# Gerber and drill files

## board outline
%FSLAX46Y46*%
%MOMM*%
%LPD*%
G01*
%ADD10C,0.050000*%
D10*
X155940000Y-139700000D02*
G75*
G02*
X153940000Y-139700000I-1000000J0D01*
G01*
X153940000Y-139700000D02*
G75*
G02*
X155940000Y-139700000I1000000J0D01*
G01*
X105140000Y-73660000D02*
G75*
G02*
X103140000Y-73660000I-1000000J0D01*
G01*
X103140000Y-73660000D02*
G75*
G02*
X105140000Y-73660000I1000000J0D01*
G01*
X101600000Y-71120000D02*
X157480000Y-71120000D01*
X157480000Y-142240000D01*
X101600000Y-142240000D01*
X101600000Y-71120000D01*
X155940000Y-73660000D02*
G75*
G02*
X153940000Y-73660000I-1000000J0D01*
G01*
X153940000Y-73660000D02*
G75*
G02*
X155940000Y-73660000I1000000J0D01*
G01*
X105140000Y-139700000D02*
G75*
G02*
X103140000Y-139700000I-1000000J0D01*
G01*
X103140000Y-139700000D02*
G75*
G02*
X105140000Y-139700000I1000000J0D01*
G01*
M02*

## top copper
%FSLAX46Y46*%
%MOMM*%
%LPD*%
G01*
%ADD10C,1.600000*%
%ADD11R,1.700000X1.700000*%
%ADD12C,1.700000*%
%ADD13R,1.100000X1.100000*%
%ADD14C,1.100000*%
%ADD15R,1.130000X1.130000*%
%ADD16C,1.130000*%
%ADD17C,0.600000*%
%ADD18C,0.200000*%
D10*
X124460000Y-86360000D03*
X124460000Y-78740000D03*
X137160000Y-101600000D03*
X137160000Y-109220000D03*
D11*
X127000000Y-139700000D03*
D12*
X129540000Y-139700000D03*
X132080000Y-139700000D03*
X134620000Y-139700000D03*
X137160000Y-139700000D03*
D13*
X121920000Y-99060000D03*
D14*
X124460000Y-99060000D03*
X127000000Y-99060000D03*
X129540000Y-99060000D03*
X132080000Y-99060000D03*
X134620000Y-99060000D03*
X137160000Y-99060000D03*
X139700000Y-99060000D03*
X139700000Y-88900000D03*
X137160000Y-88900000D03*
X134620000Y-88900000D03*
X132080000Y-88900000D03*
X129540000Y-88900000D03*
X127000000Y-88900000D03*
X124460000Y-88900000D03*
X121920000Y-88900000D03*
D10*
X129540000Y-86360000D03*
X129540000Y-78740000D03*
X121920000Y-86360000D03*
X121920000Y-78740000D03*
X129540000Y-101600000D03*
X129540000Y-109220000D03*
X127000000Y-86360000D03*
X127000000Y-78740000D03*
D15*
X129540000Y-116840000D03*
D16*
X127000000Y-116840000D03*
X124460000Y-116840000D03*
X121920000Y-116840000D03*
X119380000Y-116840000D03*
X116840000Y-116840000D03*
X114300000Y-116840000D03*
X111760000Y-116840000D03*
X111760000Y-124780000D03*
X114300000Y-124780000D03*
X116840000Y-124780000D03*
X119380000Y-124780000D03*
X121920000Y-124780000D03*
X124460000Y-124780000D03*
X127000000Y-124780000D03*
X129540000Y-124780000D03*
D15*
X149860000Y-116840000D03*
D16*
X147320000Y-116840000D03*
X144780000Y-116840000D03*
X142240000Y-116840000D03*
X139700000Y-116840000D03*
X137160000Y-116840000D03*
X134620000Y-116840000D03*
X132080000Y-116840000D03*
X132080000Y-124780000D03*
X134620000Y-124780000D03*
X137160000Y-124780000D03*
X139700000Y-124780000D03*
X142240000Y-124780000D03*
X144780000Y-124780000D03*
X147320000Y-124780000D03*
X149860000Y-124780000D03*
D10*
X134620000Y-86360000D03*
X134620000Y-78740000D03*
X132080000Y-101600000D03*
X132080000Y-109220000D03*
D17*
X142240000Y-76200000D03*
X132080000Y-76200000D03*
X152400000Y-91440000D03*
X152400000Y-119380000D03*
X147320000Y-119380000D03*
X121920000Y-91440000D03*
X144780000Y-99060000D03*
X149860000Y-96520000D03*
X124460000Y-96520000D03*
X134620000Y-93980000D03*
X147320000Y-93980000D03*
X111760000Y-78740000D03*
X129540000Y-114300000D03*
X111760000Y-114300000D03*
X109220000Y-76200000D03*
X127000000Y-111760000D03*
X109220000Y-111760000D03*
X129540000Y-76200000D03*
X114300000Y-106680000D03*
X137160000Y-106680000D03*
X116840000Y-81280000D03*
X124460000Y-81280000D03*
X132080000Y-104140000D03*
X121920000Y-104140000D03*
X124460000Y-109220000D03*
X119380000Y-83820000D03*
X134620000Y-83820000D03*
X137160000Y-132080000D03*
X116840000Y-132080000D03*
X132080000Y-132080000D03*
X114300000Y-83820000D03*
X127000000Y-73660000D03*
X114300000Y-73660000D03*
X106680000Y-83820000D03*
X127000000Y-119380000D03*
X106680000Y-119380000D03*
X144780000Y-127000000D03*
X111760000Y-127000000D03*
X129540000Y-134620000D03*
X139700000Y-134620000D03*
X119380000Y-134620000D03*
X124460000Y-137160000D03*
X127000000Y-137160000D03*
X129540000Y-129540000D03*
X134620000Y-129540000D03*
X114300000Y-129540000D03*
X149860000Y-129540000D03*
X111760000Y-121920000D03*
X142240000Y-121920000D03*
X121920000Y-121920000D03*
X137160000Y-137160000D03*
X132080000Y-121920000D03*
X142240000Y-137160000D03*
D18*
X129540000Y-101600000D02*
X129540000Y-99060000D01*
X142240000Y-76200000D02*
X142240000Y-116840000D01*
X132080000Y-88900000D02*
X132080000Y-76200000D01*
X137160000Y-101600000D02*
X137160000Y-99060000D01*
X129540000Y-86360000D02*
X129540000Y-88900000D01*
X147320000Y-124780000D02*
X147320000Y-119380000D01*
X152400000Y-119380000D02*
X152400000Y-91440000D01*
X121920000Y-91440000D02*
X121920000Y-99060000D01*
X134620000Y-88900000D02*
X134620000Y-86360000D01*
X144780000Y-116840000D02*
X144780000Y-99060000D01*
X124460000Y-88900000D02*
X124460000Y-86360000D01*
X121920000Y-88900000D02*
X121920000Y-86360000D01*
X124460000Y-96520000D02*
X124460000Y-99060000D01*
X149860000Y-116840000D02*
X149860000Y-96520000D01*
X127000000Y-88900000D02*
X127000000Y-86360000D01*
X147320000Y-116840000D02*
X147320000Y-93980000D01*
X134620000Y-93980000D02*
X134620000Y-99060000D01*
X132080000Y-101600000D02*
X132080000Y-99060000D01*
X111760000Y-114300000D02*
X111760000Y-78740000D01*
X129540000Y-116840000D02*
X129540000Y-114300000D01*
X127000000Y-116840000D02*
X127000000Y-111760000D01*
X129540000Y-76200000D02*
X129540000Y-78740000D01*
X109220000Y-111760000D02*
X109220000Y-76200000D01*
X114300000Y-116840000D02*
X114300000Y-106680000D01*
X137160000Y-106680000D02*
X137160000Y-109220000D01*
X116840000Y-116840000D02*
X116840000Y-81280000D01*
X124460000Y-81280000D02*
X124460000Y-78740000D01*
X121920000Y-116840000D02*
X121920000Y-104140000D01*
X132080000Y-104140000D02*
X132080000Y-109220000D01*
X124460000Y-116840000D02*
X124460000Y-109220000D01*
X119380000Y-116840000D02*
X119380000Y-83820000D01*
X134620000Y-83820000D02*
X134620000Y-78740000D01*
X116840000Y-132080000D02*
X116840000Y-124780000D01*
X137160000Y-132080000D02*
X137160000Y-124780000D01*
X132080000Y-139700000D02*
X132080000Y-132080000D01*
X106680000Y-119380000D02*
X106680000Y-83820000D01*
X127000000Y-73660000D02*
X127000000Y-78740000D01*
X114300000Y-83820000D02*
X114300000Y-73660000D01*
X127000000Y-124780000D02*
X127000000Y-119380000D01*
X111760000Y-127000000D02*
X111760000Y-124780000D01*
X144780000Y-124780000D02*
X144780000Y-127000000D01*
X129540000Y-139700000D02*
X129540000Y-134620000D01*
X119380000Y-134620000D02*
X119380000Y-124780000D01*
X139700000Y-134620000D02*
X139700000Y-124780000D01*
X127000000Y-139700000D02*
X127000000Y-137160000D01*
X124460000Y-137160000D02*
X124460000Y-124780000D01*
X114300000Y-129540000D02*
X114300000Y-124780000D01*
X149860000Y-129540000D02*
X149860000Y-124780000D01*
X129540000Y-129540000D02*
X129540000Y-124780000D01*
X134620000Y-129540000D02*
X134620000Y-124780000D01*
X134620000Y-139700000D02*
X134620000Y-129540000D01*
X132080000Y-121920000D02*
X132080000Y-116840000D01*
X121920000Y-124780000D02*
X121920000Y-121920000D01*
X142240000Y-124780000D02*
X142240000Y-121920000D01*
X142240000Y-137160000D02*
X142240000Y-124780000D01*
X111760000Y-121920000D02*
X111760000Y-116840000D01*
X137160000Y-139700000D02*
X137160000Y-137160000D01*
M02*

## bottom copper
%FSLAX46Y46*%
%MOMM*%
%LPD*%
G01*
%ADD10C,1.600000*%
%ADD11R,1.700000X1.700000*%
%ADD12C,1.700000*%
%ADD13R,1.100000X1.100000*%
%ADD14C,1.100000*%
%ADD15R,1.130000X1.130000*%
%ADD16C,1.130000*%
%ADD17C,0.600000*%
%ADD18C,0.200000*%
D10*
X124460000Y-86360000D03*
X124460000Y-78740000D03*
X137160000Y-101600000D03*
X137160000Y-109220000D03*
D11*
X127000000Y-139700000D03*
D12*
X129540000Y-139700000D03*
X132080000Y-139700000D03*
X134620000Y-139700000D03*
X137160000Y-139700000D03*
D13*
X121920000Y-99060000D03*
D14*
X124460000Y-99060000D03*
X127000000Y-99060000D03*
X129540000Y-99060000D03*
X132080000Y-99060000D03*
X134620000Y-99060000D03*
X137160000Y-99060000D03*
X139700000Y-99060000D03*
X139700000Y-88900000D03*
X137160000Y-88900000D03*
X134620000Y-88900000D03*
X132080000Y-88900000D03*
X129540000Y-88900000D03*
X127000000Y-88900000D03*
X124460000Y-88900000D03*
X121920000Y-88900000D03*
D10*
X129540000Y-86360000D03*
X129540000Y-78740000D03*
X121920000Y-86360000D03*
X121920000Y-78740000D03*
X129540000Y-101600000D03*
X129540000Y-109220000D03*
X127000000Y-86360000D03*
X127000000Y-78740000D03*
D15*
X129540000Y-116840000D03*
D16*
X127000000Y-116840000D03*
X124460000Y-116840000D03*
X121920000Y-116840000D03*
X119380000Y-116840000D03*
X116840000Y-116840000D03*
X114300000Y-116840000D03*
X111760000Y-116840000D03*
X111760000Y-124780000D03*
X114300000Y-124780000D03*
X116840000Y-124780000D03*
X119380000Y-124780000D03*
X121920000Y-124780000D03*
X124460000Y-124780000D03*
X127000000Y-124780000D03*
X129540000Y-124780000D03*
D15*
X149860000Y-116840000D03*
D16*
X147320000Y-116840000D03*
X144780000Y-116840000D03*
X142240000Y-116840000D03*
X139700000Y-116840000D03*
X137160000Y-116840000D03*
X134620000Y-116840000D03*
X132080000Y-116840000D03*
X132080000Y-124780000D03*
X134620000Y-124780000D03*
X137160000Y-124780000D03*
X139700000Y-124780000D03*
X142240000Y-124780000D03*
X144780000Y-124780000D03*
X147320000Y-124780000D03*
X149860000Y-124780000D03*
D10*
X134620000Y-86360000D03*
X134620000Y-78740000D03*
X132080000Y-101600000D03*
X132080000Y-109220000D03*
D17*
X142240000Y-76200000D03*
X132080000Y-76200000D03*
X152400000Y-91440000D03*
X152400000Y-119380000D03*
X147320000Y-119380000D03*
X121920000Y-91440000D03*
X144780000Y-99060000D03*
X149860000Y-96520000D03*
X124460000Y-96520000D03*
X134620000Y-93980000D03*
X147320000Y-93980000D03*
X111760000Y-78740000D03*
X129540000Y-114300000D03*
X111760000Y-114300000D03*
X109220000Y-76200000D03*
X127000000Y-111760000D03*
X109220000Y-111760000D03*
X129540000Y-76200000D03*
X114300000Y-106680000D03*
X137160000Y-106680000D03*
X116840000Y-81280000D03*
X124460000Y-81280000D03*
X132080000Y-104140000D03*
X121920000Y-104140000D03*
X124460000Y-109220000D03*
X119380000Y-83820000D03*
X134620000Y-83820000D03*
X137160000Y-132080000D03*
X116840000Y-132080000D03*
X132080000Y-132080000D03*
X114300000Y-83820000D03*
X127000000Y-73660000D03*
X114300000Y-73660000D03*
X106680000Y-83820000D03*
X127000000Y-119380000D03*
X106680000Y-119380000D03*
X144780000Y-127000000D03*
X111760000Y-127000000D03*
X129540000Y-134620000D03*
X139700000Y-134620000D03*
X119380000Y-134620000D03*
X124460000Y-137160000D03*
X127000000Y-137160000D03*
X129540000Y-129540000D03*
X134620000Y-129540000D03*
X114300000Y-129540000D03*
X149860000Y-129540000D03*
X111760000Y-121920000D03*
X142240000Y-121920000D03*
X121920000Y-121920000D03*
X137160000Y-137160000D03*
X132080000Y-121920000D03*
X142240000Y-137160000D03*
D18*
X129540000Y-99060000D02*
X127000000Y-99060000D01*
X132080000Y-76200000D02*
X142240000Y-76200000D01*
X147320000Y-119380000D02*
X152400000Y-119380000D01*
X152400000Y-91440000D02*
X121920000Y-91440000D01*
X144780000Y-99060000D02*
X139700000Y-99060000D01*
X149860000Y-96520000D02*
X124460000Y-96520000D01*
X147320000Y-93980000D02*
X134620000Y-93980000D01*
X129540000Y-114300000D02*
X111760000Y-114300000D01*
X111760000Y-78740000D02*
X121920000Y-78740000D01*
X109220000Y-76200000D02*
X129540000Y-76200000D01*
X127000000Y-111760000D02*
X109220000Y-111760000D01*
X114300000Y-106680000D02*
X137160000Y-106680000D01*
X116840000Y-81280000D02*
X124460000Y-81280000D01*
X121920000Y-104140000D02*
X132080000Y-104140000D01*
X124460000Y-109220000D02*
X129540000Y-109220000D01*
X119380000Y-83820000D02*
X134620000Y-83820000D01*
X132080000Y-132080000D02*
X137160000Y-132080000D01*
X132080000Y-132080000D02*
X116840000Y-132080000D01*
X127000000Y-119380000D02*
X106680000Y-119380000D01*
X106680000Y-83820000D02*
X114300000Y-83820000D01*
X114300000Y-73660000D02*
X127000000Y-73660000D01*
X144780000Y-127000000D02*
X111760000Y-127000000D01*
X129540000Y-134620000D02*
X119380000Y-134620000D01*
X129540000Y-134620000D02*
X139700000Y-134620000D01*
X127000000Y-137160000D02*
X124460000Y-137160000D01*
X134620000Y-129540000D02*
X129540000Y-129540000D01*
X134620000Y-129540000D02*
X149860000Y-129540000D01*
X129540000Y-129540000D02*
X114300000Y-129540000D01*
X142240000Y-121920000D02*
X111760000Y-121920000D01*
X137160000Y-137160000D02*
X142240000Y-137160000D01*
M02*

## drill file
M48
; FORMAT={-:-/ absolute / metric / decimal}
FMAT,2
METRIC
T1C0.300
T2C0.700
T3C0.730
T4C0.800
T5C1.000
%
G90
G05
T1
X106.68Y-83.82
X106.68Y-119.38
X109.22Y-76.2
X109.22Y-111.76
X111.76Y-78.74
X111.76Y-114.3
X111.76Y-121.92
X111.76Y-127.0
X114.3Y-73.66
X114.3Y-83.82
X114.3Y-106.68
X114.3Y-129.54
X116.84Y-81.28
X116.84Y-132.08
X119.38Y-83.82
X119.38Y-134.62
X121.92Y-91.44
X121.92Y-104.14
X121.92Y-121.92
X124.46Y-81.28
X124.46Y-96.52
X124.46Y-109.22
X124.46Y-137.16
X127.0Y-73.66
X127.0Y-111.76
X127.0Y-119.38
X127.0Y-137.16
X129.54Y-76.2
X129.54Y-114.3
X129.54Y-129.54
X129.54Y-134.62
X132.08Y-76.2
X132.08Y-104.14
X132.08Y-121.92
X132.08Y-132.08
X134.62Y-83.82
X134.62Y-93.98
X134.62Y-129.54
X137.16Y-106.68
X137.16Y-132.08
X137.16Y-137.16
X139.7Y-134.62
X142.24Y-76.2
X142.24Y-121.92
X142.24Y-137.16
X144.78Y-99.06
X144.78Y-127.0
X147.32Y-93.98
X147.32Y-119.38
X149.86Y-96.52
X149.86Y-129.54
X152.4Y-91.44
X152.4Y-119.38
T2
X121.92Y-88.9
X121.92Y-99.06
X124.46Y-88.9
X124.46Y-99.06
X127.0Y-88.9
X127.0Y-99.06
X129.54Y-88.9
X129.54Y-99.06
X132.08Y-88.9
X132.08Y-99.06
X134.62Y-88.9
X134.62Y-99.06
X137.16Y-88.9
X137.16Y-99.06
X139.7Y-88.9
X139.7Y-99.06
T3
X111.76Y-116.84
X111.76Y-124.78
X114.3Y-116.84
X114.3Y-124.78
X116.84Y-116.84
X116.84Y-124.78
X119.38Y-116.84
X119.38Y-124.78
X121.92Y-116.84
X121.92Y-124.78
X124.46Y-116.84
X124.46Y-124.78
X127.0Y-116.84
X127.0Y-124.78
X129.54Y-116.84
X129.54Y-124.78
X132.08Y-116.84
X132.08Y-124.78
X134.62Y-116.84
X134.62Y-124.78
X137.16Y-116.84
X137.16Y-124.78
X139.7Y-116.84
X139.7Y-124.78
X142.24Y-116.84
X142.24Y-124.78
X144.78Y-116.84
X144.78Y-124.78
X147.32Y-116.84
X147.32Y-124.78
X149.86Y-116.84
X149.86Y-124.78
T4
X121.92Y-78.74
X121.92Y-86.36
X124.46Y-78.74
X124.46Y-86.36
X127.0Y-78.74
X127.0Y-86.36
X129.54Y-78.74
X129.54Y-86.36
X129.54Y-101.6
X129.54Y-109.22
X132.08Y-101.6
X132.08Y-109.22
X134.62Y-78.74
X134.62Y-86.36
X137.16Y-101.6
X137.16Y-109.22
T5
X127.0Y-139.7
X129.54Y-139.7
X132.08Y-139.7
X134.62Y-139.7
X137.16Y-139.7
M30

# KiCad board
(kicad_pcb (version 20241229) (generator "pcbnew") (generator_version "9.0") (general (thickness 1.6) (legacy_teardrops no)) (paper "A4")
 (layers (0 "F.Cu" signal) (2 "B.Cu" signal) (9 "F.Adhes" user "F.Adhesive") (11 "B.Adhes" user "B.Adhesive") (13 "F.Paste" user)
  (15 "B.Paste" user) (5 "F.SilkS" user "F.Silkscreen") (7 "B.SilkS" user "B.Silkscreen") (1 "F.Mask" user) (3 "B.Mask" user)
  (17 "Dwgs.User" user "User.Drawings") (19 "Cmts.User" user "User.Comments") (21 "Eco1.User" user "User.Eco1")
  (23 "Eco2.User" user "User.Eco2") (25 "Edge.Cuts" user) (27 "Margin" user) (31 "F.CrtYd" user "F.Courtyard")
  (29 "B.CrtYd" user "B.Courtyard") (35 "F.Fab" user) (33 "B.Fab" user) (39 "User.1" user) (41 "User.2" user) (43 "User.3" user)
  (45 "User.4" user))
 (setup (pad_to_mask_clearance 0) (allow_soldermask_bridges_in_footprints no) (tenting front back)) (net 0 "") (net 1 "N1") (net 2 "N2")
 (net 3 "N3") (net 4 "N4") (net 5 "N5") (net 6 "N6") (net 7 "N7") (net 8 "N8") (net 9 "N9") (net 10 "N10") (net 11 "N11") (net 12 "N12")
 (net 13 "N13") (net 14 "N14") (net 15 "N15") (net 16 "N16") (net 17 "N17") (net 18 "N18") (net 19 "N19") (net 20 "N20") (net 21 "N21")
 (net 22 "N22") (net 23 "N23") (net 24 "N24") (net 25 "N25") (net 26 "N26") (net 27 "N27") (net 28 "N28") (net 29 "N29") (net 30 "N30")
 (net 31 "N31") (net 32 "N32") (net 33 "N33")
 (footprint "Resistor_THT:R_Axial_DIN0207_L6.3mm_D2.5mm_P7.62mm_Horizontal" (layer "F.Cu") (at 124.46 86.36 90)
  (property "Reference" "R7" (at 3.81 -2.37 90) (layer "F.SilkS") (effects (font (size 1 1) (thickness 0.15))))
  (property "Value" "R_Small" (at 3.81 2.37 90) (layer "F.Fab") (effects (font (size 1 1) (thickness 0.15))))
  (pad "1" thru_hole circle (at 0 0 90) (size 1.6 1.6) (drill 0.8) (layers "*.Cu" "*.Mask") (remove_unused_layers no) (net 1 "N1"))
  (pad "2" thru_hole circle (at 7.62 0 90) (size 1.6 1.6) (drill 0.8) (layers "*.Cu" "*.Mask") (remove_unused_layers no) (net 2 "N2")))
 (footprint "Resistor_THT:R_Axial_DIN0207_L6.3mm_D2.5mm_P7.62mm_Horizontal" (layer "F.Cu") (at 137.16 101.6 -90)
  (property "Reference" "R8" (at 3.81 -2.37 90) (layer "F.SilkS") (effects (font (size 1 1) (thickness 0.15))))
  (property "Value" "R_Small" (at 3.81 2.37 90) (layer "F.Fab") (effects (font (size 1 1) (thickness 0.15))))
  (pad "1" thru_hole circle (at 0 0 270) (size 1.6 1.6) (drill 0.8) (layers "*.Cu" "*.Mask") (remove_unused_layers no) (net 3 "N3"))
  (pad "2" thru_hole circle (at 7.62 0 270) (size 1.6 1.6) (drill 0.8) (layers "*.Cu" "*.Mask") (remove_unused_layers no) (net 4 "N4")))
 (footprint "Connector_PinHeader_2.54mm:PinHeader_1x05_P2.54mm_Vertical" (layer "F.Cu") (at 127 139.7 90)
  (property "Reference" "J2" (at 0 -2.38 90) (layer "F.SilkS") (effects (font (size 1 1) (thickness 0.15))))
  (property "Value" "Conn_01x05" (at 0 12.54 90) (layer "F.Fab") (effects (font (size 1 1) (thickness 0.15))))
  (pad "1" thru_hole rect (at 0 0 90) (size 1.7 1.7) (drill 1) (layers "*.Cu" "*.Mask") (remove_unused_layers no) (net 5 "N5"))
  (pad "2" thru_hole circle (at 0 2.54 90) (size 1.7 1.7) (drill 1) (layers "*.Cu" "*.Mask") (remove_unused_layers no) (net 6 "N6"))
  (pad "3" thru_hole circle (at 0 5.08 90) (size 1.7 1.7) (drill 1) (layers "*.Cu" "*.Mask") (remove_unused_layers no) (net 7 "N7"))
  (pad "4" thru_hole circle (at 0 7.62 90) (size 1.7 1.7) (drill 1) (layers "*.Cu" "*.Mask") (remove_unused_layers no) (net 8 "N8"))
  (pad "5" thru_hole circle (at 0 10.16 90) (size 1.7 1.7) (drill 1) (layers "*.Cu" "*.Mask") (remove_unused_layers no) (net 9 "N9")))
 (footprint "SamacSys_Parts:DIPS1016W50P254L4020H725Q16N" (layer "F.Cu") (at 121.92 99.06 90)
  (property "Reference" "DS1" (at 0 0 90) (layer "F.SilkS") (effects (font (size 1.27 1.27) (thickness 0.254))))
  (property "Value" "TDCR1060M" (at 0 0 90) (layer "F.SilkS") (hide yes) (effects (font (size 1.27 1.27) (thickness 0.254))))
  (pad "1" thru_hole rect (at 0 0 90) (size 1.1 1.1) (drill 0.7) (layers "*.Cu" "*.Mask") (remove_unused_layers no) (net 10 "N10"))
  (pad "2" thru_hole circle (at 0 2.54 90) (size 1.1 1.1) (drill 0.7) (layers "*.Cu" "*.Mask") (remove_unused_layers no) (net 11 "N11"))
  (pad "3" thru_hole circle (at 0 5.08 90) (size 1.1 1.1) (drill 0.7) (layers "*.Cu" "*.Mask") (remove_unused_layers no) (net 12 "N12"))
  (pad "4" thru_hole circle (at 0 7.62 90) (size 1.1 1.1) (drill 0.7) (layers "*.Cu" "*.Mask") (remove_unused_layers no) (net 12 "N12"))
  (pad "5" thru_hole circle (at 0 10.16 90) (size 1.1 1.1) (drill 0.7) (layers "*.Cu" "*.Mask") (remove_unused_layers no) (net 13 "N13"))
  (pad "6" thru_hole circle (at 0 12.7 90) (size 1.1 1.1) (drill 0.7) (layers "*.Cu" "*.Mask") (remove_unused_layers no) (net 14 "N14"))
  (pad "7" thru_hole circle (at 0 15.24 90) (size 1.1 1.1) (drill 0.7) (layers "*.Cu" "*.Mask") (remove_unused_layers no) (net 3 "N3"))
  (pad "8" thru_hole circle (at 0 17.78 90) (size 1.1 1.1) (drill 0.7) (layers "*.Cu" "*.Mask") (remove_unused_layers no) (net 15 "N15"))
  (pad "9" thru_hole circle (at 10.16 17.78 90) (size 1.1 1.1) (drill 0.7) (layers "*.Cu" "*.Mask") (remove_unused_layers no) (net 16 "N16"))
  (pad "10" thru_hole circle (at 10.16 15.24 90) (size 1.1 1.1) (drill 0.7) (layers "*.Cu" "*.Mask") (remove_unused_layers no)
   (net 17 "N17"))
  (pad "11" thru_hole circle (at 10.16 12.7 90) (size 1.1 1.1) (drill 0.7) (layers "*.Cu" "*.Mask") (remove_unused_layers no) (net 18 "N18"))
  (pad "12" thru_hole circle (at 10.16 10.16 90) (size 1.1 1.1) (drill 0.7) (layers "*.Cu" "*.Mask") (remove_unused_layers no)
   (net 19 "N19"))
  (pad "13" thru_hole circle (at 10.16 7.62 90) (size 1.1 1.1) (drill 0.7) (layers "*.Cu" "*.Mask") (remove_unused_layers no) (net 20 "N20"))
  (pad "14" thru_hole circle (at 10.16 5.08 90) (size 1.1 1.1) (drill 0.7) (layers "*.Cu" "*.Mask") (remove_unused_layers no) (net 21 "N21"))
  (pad "15" thru_hole circle (at 10.16 2.54 90) (size 1.1 1.1) (drill 0.7) (layers "*.Cu" "*.Mask") (remove_unused_layers no) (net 1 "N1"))
  (pad "16" thru_hole circle (at 10.16 0 90) (size 1.1 1.1) (drill 0.7) (layers "*.Cu" "*.Mask") (remove_unused_layers no) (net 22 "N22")))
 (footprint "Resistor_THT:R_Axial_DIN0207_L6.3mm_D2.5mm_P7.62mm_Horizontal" (layer "F.Cu") (at 129.54 86.36 90)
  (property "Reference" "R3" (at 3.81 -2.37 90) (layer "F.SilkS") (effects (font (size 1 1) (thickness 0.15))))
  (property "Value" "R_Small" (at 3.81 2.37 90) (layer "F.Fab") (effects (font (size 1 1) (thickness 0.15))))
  (pad "1" thru_hole circle (at 0 0 90) (size 1.6 1.6) (drill 0.8) (layers "*.Cu" "*.Mask") (remove_unused_layers no) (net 20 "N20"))
  (pad "2" thru_hole circle (at 7.62 0 90) (size 1.6 1.6) (drill 0.8) (layers "*.Cu" "*.Mask") (remove_unused_layers no) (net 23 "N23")))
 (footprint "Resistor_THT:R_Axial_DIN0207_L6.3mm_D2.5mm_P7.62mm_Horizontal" (layer "F.Cu") (at 121.92 86.36 90)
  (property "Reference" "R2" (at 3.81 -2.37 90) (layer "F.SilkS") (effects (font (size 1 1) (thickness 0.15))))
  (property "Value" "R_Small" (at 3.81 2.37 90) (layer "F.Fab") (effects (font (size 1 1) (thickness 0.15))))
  (pad "1" thru_hole circle (at 0 0 90) (size 1.6 1.6) (drill 0.8) (layers "*.Cu" "*.Mask") (remove_unused_layers no) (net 22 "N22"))
  (pad "2" thru_hole circle (at 7.62 0 90) (size 1.6 1.6) (drill 0.8) (layers "*.Cu" "*.Mask") (remove_unused_layers no) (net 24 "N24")))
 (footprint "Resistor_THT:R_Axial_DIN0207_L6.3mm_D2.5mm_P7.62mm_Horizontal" (layer "F.Cu") (at 129.54 101.6 -90)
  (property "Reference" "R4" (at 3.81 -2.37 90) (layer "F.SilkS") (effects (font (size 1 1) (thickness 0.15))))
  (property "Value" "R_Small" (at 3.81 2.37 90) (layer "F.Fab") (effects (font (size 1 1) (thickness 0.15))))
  (pad "1" thru_hole circle (at 0 0 270) (size 1.6 1.6) (drill 0.8) (layers "*.Cu" "*.Mask") (remove_unused_layers no) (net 12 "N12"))
  (pad "2" thru_hole circle (at 7.62 0 270) (size 1.6 1.6) (drill 0.8) (layers "*.Cu" "*.Mask") (remove_unused_layers no) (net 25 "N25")))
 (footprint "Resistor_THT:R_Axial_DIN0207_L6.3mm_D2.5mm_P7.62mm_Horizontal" (layer "F.Cu") (at 127 86.36 90)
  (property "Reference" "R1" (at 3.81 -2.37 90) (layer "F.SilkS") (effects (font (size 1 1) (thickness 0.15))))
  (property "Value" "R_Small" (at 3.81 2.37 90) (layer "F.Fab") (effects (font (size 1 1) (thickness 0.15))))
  (pad "1" thru_hole circle (at 0 0 90) (size 1.6 1.6) (drill 0.8) (layers "*.Cu" "*.Mask") (remove_unused_layers no) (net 21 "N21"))
  (pad "2" thru_hole circle (at 7.62 0 90) (size 1.6 1.6) (drill 0.8) (layers "*.Cu" "*.Mask") (remove_unused_layers no) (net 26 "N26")))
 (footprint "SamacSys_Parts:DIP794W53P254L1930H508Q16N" (layer "F.Cu") (at 120.65 120.81 -90)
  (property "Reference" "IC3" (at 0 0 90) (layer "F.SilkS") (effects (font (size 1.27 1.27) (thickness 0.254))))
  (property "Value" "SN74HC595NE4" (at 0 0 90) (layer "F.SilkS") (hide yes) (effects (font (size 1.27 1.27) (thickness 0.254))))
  (pad "1" thru_hole rect (at -3.97 -8.89 270) (size 1.13 1.13) (drill 0.73) (layers "*.Cu" "*.Mask") (remove_unused_layers no)
   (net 24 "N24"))
  (pad "2" thru_hole circle (at -3.97 -6.35 270) (size 1.13 1.13) (drill 0.73) (layers "*.Cu" "*.Mask") (remove_unused_layers no)
   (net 23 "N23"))
  (pad "3" thru_hole circle (at -3.97 -3.81 270) (size 1.13 1.13) (drill 0.73) (layers "*.Cu" "*.Mask") (remove_unused_layers no)
   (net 25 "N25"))
  (pad "4" thru_hole circle (at -3.97 -1.27 270) (size 1.13 1.13) (drill 0.73) (layers "*.Cu" "*.Mask") (remove_unused_layers no)
   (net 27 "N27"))
  (pad "5" thru_hole circle (at -3.97 1.27 270) (size 1.13 1.13) (drill 0.73) (layers "*.Cu" "*.Mask") (remove_unused_layers no)
   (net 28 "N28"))
  (pad "6" thru_hole circle (at -3.97 3.81 270) (size 1.13 1.13) (drill 0.73) (layers "*.Cu" "*.Mask") (remove_unused_layers no)
   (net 2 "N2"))
  (pad "7" thru_hole circle (at -3.97 6.35 270) (size 1.13 1.13) (drill 0.73) (layers "*.Cu" "*.Mask") (remove_unused_layers no)
   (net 4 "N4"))
  (pad "8" thru_hole circle (at -3.97 8.89 270) (size 1.13 1.13) (drill 0.73) (layers "*.Cu" "*.Mask") (remove_unused_layers no)
   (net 9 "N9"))
  (pad "9" thru_hole circle (at 3.97 8.89 270) (size 1.13 1.13) (drill 0.73) (layers "*.Cu" "*.Mask") (remove_unused_layers no)
   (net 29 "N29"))
  (pad "10" thru_hole circle (at 3.97 6.35 270) (size 1.13 1.13) (drill 0.73) (layers "*.Cu" "*.Mask") (remove_unused_layers no)
   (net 8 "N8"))
  (pad "11" thru_hole circle (at 3.97 3.81 270) (size 1.13 1.13) (drill 0.73) (layers "*.Cu" "*.Mask") (remove_unused_layers no)
   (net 7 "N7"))
  (pad "12" thru_hole circle (at 3.97 1.27 270) (size 1.13 1.13) (drill 0.73) (layers "*.Cu" "*.Mask") (remove_unused_layers no)
   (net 6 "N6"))
  (pad "13" thru_hole circle (at 3.97 -1.27 270) (size 1.13 1.13) (drill 0.73) (layers "*.Cu" "*.Mask") (remove_unused_layers no)
   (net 9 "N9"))
  (pad "14" thru_hole circle (at 3.97 -3.81 270) (size 1.13 1.13) (drill 0.73) (layers "*.Cu" "*.Mask") (remove_unused_layers no)
   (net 5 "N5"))
  (pad "15" thru_hole circle (at 3.97 -6.35 270) (size 1.13 1.13) (drill 0.73) (layers "*.Cu" "*.Mask") (remove_unused_layers no)
   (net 26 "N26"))
  (pad "16" thru_hole circle (at 3.97 -8.89 270) (size 1.13 1.13) (drill 0.73) (layers "*.Cu" "*.Mask") (remove_unused_layers no)
   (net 8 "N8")))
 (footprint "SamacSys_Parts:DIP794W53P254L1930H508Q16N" (layer "F.Cu") (at 140.97 120.81 -90)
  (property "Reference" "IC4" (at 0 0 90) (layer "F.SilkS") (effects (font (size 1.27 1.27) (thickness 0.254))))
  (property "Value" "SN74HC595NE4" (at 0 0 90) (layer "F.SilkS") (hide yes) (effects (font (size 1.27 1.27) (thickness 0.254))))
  (pad "1" thru_hole rect (at -3.97 -8.89 270) (size 1.13 1.13) (drill 0.73) (layers "*.Cu" "*.Mask") (remove_unused_layers no)
   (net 11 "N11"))
  (pad "2" thru_hole circle (at -3.97 -6.35 270) (size 1.13 1.13) (drill 0.73) (layers "*.Cu" "*.Mask") (remove_unused_layers no)
   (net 14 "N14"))
  (pad "3" thru_hole circle (at -3.97 -3.81 270) (size 1.13 1.13) (drill 0.73) (layers "*.Cu" "*.Mask") (remove_unused_layers no)
   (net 15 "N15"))
  (pad "4" thru_hole circle (at -3.97 -1.27 270) (size 1.13 1.13) (drill 0.73) (layers "*.Cu" "*.Mask") (remove_unused_layers no)
   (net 19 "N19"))
  (pad "5" thru_hole circle (at -3.97 1.27 270) (size 1.13 1.13) (drill 0.73) (layers "*.Cu" "*.Mask") (remove_unused_layers no)
   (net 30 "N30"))
  (pad "6" thru_hole circle (at -3.97 3.81 270) (size 1.13 1.13) (drill 0.73) (layers "*.Cu" "*.Mask") (remove_unused_layers no)
   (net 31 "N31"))
  (pad "7" thru_hole circle (at -3.97 6.35 270) (size 1.13 1.13) (drill 0.73) (layers "*.Cu" "*.Mask") (remove_unused_layers no)
   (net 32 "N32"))
  (pad "8" thru_hole circle (at -3.97 8.89 270) (size 1.13 1.13) (drill 0.73) (layers "*.Cu" "*.Mask") (remove_unused_layers no)
   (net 9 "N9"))
  (pad "9" thru_hole circle (at 3.97 8.89 270) (size 1.13 1.13) (drill 0.73) (layers "*.Cu" "*.Mask") (remove_unused_layers no)
   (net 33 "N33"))
  (pad "10" thru_hole circle (at 3.97 6.35 270) (size 1.13 1.13) (drill 0.73) (layers "*.Cu" "*.Mask") (remove_unused_layers no)
   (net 8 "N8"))
  (pad "11" thru_hole circle (at 3.97 3.81 270) (size 1.13 1.13) (drill 0.73) (layers "*.Cu" "*.Mask") (remove_unused_layers no)
   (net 7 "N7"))
  (pad "12" thru_hole circle (at 3.97 1.27 270) (size 1.13 1.13) (drill 0.73) (layers "*.Cu" "*.Mask") (remove_unused_layers no)
   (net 6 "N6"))
  (pad "13" thru_hole circle (at 3.97 -1.27 270) (size 1.13 1.13) (drill 0.73) (layers "*.Cu" "*.Mask") (remove_unused_layers no)
   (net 9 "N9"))
  (pad "14" thru_hole circle (at 3.97 -3.81 270) (size 1.13 1.13) (drill 0.73) (layers "*.Cu" "*.Mask") (remove_unused_layers no)
   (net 29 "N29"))
  (pad "15" thru_hole circle (at 3.97 -6.35 270) (size 1.13 1.13) (drill 0.73) (layers "*.Cu" "*.Mask") (remove_unused_layers no)
   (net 10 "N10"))
  (pad "16" thru_hole circle (at 3.97 -8.89 270) (size 1.13 1.13) (drill 0.73) (layers "*.Cu" "*.Mask") (remove_unused_layers no)
   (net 8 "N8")))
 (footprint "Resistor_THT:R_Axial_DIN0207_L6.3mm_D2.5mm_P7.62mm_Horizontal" (layer "F.Cu") (at 134.62 86.36 90)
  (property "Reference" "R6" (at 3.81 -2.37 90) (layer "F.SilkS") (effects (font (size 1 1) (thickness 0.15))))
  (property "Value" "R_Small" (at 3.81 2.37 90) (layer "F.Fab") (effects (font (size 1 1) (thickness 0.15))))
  (pad "1" thru_hole circle (at 0 0 90) (size 1.6 1.6) (drill 0.8) (layers "*.Cu" "*.Mask") (remove_unused_layers no) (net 18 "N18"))
  (pad "2" thru_hole circle (at 7.62 0 90) (size 1.6 1.6) (drill 0.8) (layers "*.Cu" "*.Mask") (remove_unused_layers no) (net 28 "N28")))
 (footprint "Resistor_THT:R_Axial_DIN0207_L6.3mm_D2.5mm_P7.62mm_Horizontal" (layer "F.Cu") (at 132.08 101.6 -90)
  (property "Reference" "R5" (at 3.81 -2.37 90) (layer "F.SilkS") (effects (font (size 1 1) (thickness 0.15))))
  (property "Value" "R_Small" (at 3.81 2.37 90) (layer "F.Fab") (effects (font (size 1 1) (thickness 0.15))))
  (pad "1" thru_hole circle (at 0 0 270) (size 1.6 1.6) (drill 0.8) (layers "*.Cu" "*.Mask") (remove_unused_layers no) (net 13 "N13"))
  (pad "2" thru_hole circle (at 7.62 0 270) (size 1.6 1.6) (drill 0.8) (layers "*.Cu" "*.Mask") (remove_unused_layers no) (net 27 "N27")))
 (gr_circle (center 154.94 139.7) (end 155.94 139.7) (stroke (width 0.05) (type default)) (fill no) (layer "Edge.Cuts"))
 (gr_circle (center 104.14 73.66) (end 105.14 73.66) (stroke (width 0.05) (type default)) (fill no) (layer "Edge.Cuts"))
 (gr_rect (start 101.6 71.12) (end 157.48 142.24) (stroke (width 0.05) (type default)) (fill no) (layer "Edge.Cuts"))
 (gr_circle (center 154.94 73.66) (end 155.94 73.66) (stroke (width 0.05) (type default)) (fill no) (layer "Edge.Cuts"))
 (gr_circle (center 104.14 139.7) (end 105.14 139.7) (stroke (width 0.05) (type default)) (fill no) (layer "Edge.Cuts"))
 (segment (start 129.54 101.6) (end 129.54 99.06) (width 0.2) (layer "F.Cu") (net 12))
 (segment (start 129.54 99.06) (end 127 99.06) (width 0.2) (layer "B.Cu") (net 12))
 (segment (start 142.24 76.2) (end 142.24 116.84) (width 0.2) (layer "F.Cu") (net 19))
 (segment (start 132.08 88.9) (end 132.08 76.2) (width 0.2) (layer "F.Cu") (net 19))
 (via (at 142.24 76.2) (size 0.6) (drill 0.3) (layers "F.Cu" "B.Cu") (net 19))
 (via (at 132.08 76.2) (size 0.6) (drill 0.3) (layers "F.Cu" "B.Cu") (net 19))
 (segment (start 132.08 76.2) (end 142.24 76.2) (width 0.2) (layer "B.Cu") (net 19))
 (segment (start 137.16 101.6) (end 137.16 99.06) (width 0.2) (layer "F.Cu") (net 3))
 (segment (start 129.54 86.36) (end 129.54 88.9) (width 0.2) (layer "F.Cu") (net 20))
 (segment (start 147.32 124.78) (end 147.32 119.38) (width 0.2) (layer "F.Cu") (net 10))
 (segment (start 152.4 119.38) (end 152.4 91.44) (width 0.2) (layer "F.Cu") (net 10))
 (segment (start 121.92 91.44) (end 121.92 99.06) (width 0.2) (layer "F.Cu") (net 10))
 (via (at 152.4 91.44) (size 0.6) (drill 0.3) (layers "F.Cu" "B.Cu") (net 10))
 (via (at 152.4 119.38) (size 0.6) (drill 0.3) (layers "F.Cu" "B.Cu") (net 10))
 (via (at 147.32 119.38) (size 0.6) (drill 0.3) (layers "F.Cu" "B.Cu") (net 10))
 (via (at 121.92 91.44) (size 0.6) (drill 0.3) (layers "F.Cu" "B.Cu") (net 10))
 (segment (start 147.32 119.38) (end 152.4 119.38) (width 0.2) (layer "B.Cu") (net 10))
 (segment (start 152.4 91.44) (end 121.92 91.44) (width 0.2) (layer "B.Cu") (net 10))
 (segment (start 134.62 88.9) (end 134.62 86.36) (width 0.2) (layer "F.Cu") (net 18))
 (segment (start 144.78 116.84) (end 144.78 99.06) (width 0.2) (layer "F.Cu") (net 15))
 (via (at 144.78 99.06) (size 0.6) (drill 0.3) (layers "F.Cu" "B.Cu") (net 15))
 (segment (start 144.78 99.06) (end 139.7 99.06) (width 0.2) (layer "B.Cu") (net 15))
 (segment (start 124.46 88.9) (end 124.46 86.36) (width 0.2) (layer "F.Cu") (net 1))
 (segment (start 121.92 88.9) (end 121.92 86.36) (width 0.2) (layer "F.Cu") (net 22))
 (segment (start 124.46 96.52) (end 124.46 99.06) (width 0.2) (layer "F.Cu") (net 11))
 (segment (start 149.86 116.84) (end 149.86 96.52) (width 0.2) (layer "F.Cu") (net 11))
 (via (at 149.86 96.52) (size 0.6) (drill 0.3) (layers "F.Cu" "B.Cu") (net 11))
 (via (at 124.46 96.52) (size 0.6) (drill 0.3) (layers "F.Cu" "B.Cu") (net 11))
 (segment (start 149.86 96.52) (end 124.46 96.52) (width 0.2) (layer "B.Cu") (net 11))
 (segment (start 127 88.9) (end 127 86.36) (width 0.2) (layer "F.Cu") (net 21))
 (segment (start 147.32 116.84) (end 147.32 93.98) (width 0.2) (layer "F.Cu") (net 14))
 (segment (start 134.62 93.98) (end 134.62 99.06) (width 0.2) (layer "F.Cu") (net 14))
 (via (at 134.62 93.98) (size 0.6) (drill 0.3) (layers "F.Cu" "B.Cu") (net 14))
 (via (at 147.32 93.98) (size 0.6) (drill 0.3) (layers "F.Cu" "B.Cu") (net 14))
 (segment (start 147.32 93.98) (end 134.62 93.98) (width 0.2) (layer "B.Cu") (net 14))
 (segment (start 132.08 101.6) (end 132.08 99.06) (width 0.2) (layer "F.Cu") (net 13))
 (segment (start 111.76 114.3) (end 111.76 78.74) (width 0.2) (layer "F.Cu") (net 24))
 (segment (start 129.54 116.84) (end 129.54 114.3) (width 0.2) (layer "F.Cu") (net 24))
 (via (at 111.76 78.74) (size 0.6) (drill 0.3) (layers "F.Cu" "B.Cu") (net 24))
 (via (at 129.54 114.3) (size 0.6) (drill 0.3) (layers "F.Cu" "B.Cu") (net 24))
 (via (at 111.76 114.3) (size 0.6) (drill 0.3) (layers "F.Cu" "B.Cu") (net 24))
 (segment (start 129.54 114.3) (end 111.76 114.3) (width 0.2) (layer "B.Cu") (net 24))
 (segment (start 111.76 78.74) (end 121.92 78.74) (width 0.2) (layer "B.Cu") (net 24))
 (segment (start 127 116.84) (end 127 111.76) (width 0.2) (layer "F.Cu") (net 23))
 (segment (start 129.54 76.2) (end 129.54 78.74) (width 0.2) (layer "F.Cu") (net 23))
 (segment (start 109.22 111.76) (end 109.22 76.2) (width 0.2) (layer "F.Cu") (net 23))
 (via (at 109.22 76.2) (size 0.6) (drill 0.3) (layers "F.Cu" "B.Cu") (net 23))
 (via (at 127 111.76) (size 0.6) (drill 0.3) (layers "F.Cu" "B.Cu") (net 23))
 (via (at 109.22 111.76) (size 0.6) (drill 0.3) (layers "F.Cu" "B.Cu") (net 23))
 (via (at 129.54 76.2) (size 0.6) (drill 0.3) (layers "F.Cu" "B.Cu") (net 23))
 (segment (start 109.22 76.2) (end 129.54 76.2) (width 0.2) (layer "B.Cu") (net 23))
 (segment (start 127 111.76) (end 109.22 111.76) (width 0.2) (layer "B.Cu") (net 23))
 (segment (start 114.3 116.84) (end 114.3 106.68) (width 0.2) (layer "F.Cu") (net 4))
 (segment (start 137.16 106.68) (end 137.16 109.22) (width 0.2) (layer "F.Cu") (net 4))
 (via (at 114.3 106.68) (size 0.6) (drill 0.3) (layers "F.Cu" "B.Cu") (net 4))
 (via (at 137.16 106.68) (size 0.6) (drill 0.3) (layers "F.Cu" "B.Cu") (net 4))
 (segment (start 114.3 106.68) (end 137.16 106.68) (width 0.2) (layer "B.Cu") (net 4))
 (segment (start 116.84 116.84) (end 116.84 81.28) (width 0.2) (layer "F.Cu") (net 2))
 (segment (start 124.46 81.28) (end 124.46 78.74) (width 0.2) (layer "F.Cu") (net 2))
 (via (at 116.84 81.28) (size 0.6) (drill 0.3) (layers "F.Cu" "B.Cu") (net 2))
 (via (at 124.46 81.28) (size 0.6) (drill 0.3) (layers "F.Cu" "B.Cu") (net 2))
 (segment (start 116.84 81.28) (end 124.46 81.28) (width 0.2) (layer "B.Cu") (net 2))
 (segment (start 121.92 116.84) (end 121.92 104.14) (width 0.2) (layer "F.Cu") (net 27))
 (segment (start 132.08 104.14) (end 132.08 109.22) (width 0.2) (layer "F.Cu") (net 27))
 (via (at 132.08 104.14) (size 0.6) (drill 0.3) (layers "F.Cu" "B.Cu") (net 27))
 (via (at 121.92 104.14) (size 0.6) (drill 0.3) (layers "F.Cu" "B.Cu") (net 27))
 (segment (start 121.92 104.14) (end 132.08 104.14) (width 0.2) (layer "B.Cu") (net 27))
 (segment (start 124.46 116.84) (end 124.46 109.22) (width 0.2) (layer "F.Cu") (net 25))
 (via (at 124.46 109.22) (size 0.6) (drill 0.3) (layers "F.Cu" "B.Cu") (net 25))
 (segment (start 124.46 109.22) (end 129.54 109.22) (width 0.2) (layer "B.Cu") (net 25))
 (segment (start 119.38 116.84) (end 119.38 83.82) (width 0.2) (layer "F.Cu") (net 28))
 (segment (start 134.62 83.82) (end 134.62 78.74) (width 0.2) (layer "F.Cu") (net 28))
 (via (at 119.38 83.82) (size 0.6) (drill 0.3) (layers "F.Cu" "B.Cu") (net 28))
 (via (at 134.62 83.82) (size 0.6) (drill 0.3) (layers "F.Cu" "B.Cu") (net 28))
 (segment (start 119.38 83.82) (end 134.62 83.82) (width 0.2) (layer "B.Cu") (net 28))
 (segment (start 116.84 132.08) (end 116.84 124.78) (width 0.2) (layer "F.Cu") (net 7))
 (segment (start 137.16 132.08) (end 137.16 124.78) (width 0.2) (layer "F.Cu") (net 7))
 (segment (start 132.08 139.7) (end 132.08 132.08) (width 0.2) (layer "F.Cu") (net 7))
 (via (at 137.16 132.08) (size 0.6) (drill 0.3) (layers "F.Cu" "B.Cu") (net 7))
 (via (at 116.84 132.08) (size 0.6) (drill 0.3) (layers "F.Cu" "B.Cu") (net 7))
 (via (at 132.08 132.08) (size 0.6) (drill 0.3) (layers "F.Cu" "B.Cu") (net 7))
 (segment (start 132.08 132.08) (end 137.16 132.08) (width 0.2) (layer "B.Cu") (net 7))
 (segment (start 132.08 132.08) (end 116.84 132.08) (width 0.2) (layer "B.Cu") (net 7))
 (segment (start 106.68 119.38) (end 106.68 83.82) (width 0.2) (layer "F.Cu") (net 26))
 (segment (start 127 73.66) (end 127 78.74) (width 0.2) (layer "F.Cu") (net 26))
 (segment (start 114.3 83.82) (end 114.3 73.66) (width 0.2) (layer "F.Cu") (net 26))
 (segment (start 127 124.78) (end 127 119.38) (width 0.2) (layer "F.Cu") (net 26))
 (via (at 114.3 83.82) (size 0.6) (drill 0.3) (layers "F.Cu" "B.Cu") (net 26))
 (via (at 127 73.66) (size 0.6) (drill 0.3) (layers "F.Cu" "B.Cu") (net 26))
 (via (at 114.3 73.66) (size 0.6) (drill 0.3) (layers "F.Cu" "B.Cu") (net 26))
 (via (at 106.68 83.82) (size 0.6) (drill 0.3) (layers "F.Cu" "B.Cu") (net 26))
 (via (at 127 119.38) (size 0.6) (drill 0.3) (layers "F.Cu" "B.Cu") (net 26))
 (via (at 106.68 119.38) (size 0.6) (drill 0.3) (layers "F.Cu" "B.Cu") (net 26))
 (segment (start 127 119.38) (end 106.68 119.38) (width 0.2) (layer "B.Cu") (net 26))
 (segment (start 106.68 83.82) (end 114.3 83.82) (width 0.2) (layer "B.Cu") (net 26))
 (segment (start 114.3 73.66) (end 127 73.66) (width 0.2) (layer "B.Cu") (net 26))
 (segment (start 111.76 127) (end 111.76 124.78) (width 0.2) (layer "F.Cu") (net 29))
 (segment (start 144.78 124.78) (end 144.78 127) (width 0.2) (layer "F.Cu") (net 29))
 (via (at 144.78 127) (size 0.6) (drill 0.3) (layers "F.Cu" "B.Cu") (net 29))
 (via (at 111.76 127) (size 0.6) (drill 0.3) (layers "F.Cu" "B.Cu") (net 29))
 (segment (start 144.78 127) (end 111.76 127) (width 0.2) (layer "B.Cu") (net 29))
 (segment (start 129.54 139.7) (end 129.54 134.62) (width 0.2) (layer "F.Cu") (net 6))
 (segment (start 119.38 134.62) (end 119.38 124.78) (width 0.2) (layer "F.Cu") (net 6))
 (segment (start 139.7 134.62) (end 139.7 124.78) (width 0.2) (layer "F.Cu") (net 6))
 (via (at 129.54 134.62) (size 0.6) (drill 0.3) (layers "F.Cu" "B.Cu") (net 6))
 (via (at 139.7 134.62) (size 0.6) (drill 0.3) (layers "F.Cu" "B.Cu") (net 6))
 (via (at 119.38 134.62) (size 0.6) (drill 0.3) (layers "F.Cu" "B.Cu") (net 6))
 (segment (start 129.54 134.62) (end 119.38 134.62) (width 0.2) (layer "B.Cu") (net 6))
 (segment (start 129.54 134.62) (end 139.7 134.62) (width 0.2) (layer "B.Cu") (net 6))
 (segment (start 127 139.7) (end 127 137.16) (width 0.2) (layer "F.Cu") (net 5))
 (segment (start 124.46 137.16) (end 124.46 124.78) (width 0.2) (layer "F.Cu") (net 5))
 (via (at 124.46 137.16) (size 0.6) (drill 0.3) (layers "F.Cu" "B.Cu") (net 5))
 (via (at 127 137.16) (size 0.6) (drill 0.3) (layers "F.Cu" "B.Cu") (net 5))
 (segment (start 127 137.16) (end 124.46 137.16) (width 0.2) (layer "B.Cu") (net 5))
 (segment (start 114.3 129.54) (end 114.3 124.78) (width 0.2) (layer "F.Cu") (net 8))
 (segment (start 149.86 129.54) (end 149.86 124.78) (width 0.2) (layer "F.Cu") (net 8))
 (segment (start 129.54 129.54) (end 129.54 124.78) (width 0.2) (layer "F.Cu") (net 8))
 (segment (start 134.62 129.54) (end 134.62 124.78) (width 0.2) (layer "F.Cu") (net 8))
 (segment (start 134.62 139.7) (end 134.62 129.54) (width 0.2) (layer "F.Cu") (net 8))
 (via (at 129.54 129.54) (size 0.6) (drill 0.3) (layers "F.Cu" "B.Cu") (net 8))
 (via (at 134.62 129.54) (size 0.6) (drill 0.3) (layers "F.Cu" "B.Cu") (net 8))
 (via (at 114.3 129.54) (size 0.6) (drill 0.3) (layers "F.Cu" "B.Cu") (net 8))
 (via (at 149.86 129.54) (size 0.6) (drill 0.3) (layers "F.Cu" "B.Cu") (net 8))
 (segment (start 134.62 129.54) (end 129.54 129.54) (width 0.2) (layer "B.Cu") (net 8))
 (segment (start 134.62 129.54) (end 149.86 129.54) (width 0.2) (layer "B.Cu") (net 8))
 (segment (start 129.54 129.54) (end 114.3 129.54) (width 0.2) (layer "B.Cu") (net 8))
 (segment (start 132.08 121.92) (end 132.08 116.84) (width 0.2) (layer "F.Cu") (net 9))
 (segment (start 121.92 124.78) (end 121.92 121.92) (width 0.2) (layer "F.Cu") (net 9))
 (segment (start 142.24 124.78) (end 142.24 121.92) (width 0.2) (layer "F.Cu") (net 9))
 (segment (start 142.24 137.16) (end 142.24 124.78) (width 0.2) (layer "F.Cu") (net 9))
 (segment (start 111.76 121.92) (end 111.76 116.84) (width 0.2) (layer "F.Cu") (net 9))
 (segment (start 137.16 139.7) (end 137.16 137.16) (width 0.2) (layer "F.Cu") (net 9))
 (via (at 111.76 121.92) (size 0.6) (drill 0.3) (layers "F.Cu" "B.Cu") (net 9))
 (via (at 142.24 121.92) (size 0.6) (drill 0.3) (layers "F.Cu" "B.Cu") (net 9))
 (via (at 121.92 121.92) (size 0.6) (drill 0.3) (layers "F.Cu" "B.Cu") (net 9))
 (via (at 137.16 137.16) (size 0.6) (drill 0.3) (layers "F.Cu" "B.Cu") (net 9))
 (via (at 132.08 121.92) (size 0.6) (drill 0.3) (layers "F.Cu" "B.Cu") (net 9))
 (via (at 142.24 137.16) (size 0.6) (drill 0.3) (layers "F.Cu" "B.Cu") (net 9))
 (segment (start 142.24 121.92) (end 111.76 121.92) (width 0.2) (layer "B.Cu") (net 9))
 (segment (start 137.16 137.16) (end 142.24 137.16) (width 0.2) (layer "B.Cu") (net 9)))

